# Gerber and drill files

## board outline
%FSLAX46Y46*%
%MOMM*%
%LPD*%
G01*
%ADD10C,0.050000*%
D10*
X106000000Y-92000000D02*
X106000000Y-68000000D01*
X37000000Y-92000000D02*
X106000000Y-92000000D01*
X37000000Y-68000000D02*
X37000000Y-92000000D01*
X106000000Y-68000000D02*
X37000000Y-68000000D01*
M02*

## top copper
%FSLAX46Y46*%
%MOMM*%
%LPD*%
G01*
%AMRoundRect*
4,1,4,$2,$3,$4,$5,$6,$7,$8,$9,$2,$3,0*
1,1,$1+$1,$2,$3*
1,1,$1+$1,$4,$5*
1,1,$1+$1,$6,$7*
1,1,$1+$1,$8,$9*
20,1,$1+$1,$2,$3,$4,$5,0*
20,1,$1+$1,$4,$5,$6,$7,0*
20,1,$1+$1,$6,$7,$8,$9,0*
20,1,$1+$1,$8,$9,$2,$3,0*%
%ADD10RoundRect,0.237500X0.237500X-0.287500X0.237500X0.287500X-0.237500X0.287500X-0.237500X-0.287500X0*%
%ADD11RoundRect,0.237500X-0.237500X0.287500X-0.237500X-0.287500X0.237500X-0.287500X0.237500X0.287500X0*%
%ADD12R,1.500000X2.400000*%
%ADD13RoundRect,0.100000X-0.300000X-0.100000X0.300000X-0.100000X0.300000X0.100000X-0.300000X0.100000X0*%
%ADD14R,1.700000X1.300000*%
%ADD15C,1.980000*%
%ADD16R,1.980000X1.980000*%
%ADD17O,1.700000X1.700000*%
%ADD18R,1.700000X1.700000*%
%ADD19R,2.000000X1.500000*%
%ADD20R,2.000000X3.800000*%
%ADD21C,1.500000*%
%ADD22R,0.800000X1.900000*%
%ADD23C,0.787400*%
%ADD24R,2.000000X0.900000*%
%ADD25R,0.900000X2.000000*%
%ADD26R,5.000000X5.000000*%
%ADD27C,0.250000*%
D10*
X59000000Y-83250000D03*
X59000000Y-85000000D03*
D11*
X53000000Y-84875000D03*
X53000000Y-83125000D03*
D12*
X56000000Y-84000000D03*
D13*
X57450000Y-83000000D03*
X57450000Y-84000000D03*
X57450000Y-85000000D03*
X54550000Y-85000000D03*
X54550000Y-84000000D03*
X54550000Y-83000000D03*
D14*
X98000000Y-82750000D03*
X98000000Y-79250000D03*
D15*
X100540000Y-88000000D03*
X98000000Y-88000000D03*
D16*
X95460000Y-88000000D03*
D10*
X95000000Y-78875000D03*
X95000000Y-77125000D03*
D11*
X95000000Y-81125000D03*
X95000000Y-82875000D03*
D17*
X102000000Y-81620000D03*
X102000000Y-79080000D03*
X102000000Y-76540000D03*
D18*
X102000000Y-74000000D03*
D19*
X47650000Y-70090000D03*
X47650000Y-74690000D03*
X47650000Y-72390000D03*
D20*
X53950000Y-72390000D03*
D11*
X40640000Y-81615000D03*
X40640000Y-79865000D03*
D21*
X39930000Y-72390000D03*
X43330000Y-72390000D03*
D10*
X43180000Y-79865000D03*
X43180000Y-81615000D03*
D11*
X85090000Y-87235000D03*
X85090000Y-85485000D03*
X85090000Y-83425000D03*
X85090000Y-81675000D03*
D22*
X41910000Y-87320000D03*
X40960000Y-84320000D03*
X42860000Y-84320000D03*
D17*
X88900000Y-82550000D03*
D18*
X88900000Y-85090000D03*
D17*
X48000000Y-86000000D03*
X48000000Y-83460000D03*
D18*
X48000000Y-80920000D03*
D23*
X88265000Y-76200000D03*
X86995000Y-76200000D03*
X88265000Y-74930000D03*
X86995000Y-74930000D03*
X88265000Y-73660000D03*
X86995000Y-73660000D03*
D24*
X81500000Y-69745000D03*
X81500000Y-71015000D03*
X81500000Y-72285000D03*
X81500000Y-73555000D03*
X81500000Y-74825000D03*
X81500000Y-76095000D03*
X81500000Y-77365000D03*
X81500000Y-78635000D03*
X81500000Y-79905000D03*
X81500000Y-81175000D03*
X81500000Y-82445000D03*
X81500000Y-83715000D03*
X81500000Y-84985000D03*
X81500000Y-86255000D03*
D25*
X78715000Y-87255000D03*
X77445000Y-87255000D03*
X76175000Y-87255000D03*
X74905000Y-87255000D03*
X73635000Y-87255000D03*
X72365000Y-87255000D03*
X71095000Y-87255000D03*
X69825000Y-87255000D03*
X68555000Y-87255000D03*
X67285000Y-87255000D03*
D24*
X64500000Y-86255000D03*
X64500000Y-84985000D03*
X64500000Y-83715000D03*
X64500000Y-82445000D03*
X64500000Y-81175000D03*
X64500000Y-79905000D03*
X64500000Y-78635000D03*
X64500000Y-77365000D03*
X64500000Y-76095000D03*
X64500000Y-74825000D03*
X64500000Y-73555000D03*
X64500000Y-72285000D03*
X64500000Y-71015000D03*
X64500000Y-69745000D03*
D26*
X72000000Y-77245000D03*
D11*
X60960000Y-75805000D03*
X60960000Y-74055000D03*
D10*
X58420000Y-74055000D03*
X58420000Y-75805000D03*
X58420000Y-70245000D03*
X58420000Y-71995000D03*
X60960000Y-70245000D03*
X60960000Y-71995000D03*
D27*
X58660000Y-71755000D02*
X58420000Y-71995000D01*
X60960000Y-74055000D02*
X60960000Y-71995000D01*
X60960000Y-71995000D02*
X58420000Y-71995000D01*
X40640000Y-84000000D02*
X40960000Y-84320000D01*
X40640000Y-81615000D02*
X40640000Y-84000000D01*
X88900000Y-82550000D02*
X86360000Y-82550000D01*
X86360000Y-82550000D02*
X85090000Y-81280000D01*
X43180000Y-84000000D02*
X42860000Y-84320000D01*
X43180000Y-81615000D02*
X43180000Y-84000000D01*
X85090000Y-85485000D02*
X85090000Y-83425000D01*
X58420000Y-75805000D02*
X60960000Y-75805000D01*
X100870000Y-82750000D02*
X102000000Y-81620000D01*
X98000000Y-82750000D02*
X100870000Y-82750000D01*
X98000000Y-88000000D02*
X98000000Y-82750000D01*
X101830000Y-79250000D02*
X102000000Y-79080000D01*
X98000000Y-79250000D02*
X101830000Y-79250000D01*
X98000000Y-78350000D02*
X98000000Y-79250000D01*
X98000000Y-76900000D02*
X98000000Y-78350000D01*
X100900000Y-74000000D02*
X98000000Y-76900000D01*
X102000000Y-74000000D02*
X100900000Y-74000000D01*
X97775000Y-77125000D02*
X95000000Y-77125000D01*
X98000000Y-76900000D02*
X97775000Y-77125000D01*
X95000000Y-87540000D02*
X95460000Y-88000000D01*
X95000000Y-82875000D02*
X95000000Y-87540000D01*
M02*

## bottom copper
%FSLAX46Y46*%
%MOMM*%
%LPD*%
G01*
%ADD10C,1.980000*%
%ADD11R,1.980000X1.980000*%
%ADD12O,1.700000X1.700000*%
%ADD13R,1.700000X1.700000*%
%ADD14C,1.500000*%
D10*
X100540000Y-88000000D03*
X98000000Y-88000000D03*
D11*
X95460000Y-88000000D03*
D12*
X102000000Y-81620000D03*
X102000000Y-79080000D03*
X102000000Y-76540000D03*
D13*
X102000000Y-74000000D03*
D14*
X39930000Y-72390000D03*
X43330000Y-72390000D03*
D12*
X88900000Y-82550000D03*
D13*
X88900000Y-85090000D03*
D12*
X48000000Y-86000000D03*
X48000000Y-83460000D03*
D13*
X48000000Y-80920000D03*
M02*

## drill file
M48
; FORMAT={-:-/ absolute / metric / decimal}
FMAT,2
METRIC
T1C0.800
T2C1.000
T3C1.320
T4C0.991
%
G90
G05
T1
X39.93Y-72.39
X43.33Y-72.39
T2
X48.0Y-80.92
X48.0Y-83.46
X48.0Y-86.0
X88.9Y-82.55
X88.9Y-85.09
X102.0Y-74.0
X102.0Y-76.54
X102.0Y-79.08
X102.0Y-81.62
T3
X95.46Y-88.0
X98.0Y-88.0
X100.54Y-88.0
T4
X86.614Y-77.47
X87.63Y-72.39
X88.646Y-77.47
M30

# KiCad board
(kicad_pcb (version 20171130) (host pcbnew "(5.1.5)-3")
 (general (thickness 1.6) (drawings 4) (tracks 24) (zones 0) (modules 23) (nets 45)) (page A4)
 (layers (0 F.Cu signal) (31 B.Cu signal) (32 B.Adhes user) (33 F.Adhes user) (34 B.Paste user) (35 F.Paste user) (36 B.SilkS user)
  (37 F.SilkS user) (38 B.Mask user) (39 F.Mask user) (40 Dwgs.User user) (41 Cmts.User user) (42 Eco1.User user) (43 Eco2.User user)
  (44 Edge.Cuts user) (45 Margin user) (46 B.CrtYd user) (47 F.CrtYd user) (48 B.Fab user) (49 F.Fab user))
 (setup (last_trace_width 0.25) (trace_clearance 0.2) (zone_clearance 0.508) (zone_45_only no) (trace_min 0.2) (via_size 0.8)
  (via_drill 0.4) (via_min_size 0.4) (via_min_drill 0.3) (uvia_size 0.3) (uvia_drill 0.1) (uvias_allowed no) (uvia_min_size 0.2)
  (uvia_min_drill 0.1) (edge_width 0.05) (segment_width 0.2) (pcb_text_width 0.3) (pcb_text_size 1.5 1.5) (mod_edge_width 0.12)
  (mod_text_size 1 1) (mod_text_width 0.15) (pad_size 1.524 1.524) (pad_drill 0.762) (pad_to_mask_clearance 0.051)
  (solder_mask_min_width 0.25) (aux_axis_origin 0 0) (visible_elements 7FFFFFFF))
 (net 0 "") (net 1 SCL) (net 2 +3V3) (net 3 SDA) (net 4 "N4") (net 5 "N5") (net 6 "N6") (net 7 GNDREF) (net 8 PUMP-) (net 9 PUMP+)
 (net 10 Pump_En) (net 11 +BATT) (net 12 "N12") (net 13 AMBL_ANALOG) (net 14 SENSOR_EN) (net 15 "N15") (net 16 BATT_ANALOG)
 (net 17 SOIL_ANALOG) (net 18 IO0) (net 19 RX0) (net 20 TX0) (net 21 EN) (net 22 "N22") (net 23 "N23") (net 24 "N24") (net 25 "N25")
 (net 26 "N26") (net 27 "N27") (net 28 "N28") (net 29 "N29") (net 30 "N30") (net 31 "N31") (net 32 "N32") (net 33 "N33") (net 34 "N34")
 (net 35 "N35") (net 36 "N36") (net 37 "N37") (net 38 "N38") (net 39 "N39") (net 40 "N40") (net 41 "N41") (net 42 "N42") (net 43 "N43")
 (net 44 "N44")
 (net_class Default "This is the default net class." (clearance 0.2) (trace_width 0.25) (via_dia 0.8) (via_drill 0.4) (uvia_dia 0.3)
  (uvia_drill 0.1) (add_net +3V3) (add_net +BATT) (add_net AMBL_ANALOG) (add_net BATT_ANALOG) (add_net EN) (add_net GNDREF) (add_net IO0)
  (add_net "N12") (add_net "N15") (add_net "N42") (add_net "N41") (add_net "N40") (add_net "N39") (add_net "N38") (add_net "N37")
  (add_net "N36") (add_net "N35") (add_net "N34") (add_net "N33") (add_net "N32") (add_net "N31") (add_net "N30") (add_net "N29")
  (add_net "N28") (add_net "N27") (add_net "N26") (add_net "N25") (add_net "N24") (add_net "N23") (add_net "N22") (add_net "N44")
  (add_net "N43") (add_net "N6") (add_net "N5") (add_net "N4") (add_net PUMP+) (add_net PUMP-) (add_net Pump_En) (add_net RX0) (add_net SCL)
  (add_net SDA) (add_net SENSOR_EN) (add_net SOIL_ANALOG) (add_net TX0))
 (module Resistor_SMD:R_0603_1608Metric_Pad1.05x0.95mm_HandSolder (layer F.Cu) (at 59 84.125 90)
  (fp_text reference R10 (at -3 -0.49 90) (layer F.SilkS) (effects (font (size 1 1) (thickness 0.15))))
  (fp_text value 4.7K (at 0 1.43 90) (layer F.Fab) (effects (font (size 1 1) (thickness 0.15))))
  (pad 2 smd roundrect (at 0.875 0 90) (size 1.05 0.95) (layers F.Cu F.Paste F.Mask) (roundrect_rratio 0.25) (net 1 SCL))
  (pad 1 smd roundrect (at -0.875 0 90) (size 1.05 0.95) (layers F.Cu F.Paste F.Mask) (roundrect_rratio 0.25) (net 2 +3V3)))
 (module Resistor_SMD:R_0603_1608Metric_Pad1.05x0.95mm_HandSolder (layer F.Cu) (at 53 84 270)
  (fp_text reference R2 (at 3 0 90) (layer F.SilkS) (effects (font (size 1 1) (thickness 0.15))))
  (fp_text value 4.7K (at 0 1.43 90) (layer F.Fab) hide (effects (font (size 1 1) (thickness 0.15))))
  (pad 2 smd roundrect (at 0.875 0 270) (size 1.05 0.95) (layers F.Cu F.Paste F.Mask) (roundrect_rratio 0.25) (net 2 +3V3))
  (pad 1 smd roundrect (at -0.875 0 270) (size 1.05 0.95) (layers F.Cu F.Paste F.Mask) (roundrect_rratio 0.25) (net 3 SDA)))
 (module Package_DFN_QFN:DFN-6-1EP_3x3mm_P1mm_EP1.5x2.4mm (layer F.Cu) (at 56 84)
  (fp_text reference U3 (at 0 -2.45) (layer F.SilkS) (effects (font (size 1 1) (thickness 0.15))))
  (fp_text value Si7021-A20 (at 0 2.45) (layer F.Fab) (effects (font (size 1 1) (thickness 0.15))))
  (pad "" smd roundrect (at 0.375 0.6) (size 0.6 0.97) (layers F.Paste) (roundrect_rratio 0.25))
  (pad "" smd roundrect (at 0.375 -0.6) (size 0.6 0.97) (layers F.Paste) (roundrect_rratio 0.25))
  (pad "" smd roundrect (at -0.375 0.6) (size 0.6 0.97) (layers F.Paste) (roundrect_rratio 0.25))
  (pad "" smd roundrect (at -0.375 -0.6) (size 0.6 0.97) (layers F.Paste) (roundrect_rratio 0.25))
  (pad 7 smd rect (at 0 0) (size 1.5 2.4) (layers F.Cu F.Mask) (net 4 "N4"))
  (pad 6 smd roundrect (at 1.45 -1) (size 0.8 0.4) (layers F.Cu F.Paste F.Mask) (roundrect_rratio 0.25) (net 1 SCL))
  (pad 5 smd roundrect (at 1.45 0) (size 0.8 0.4) (layers F.Cu F.Paste F.Mask) (roundrect_rratio 0.25) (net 2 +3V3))
  (pad 4 smd roundrect (at 1.45 1) (size 0.8 0.4) (layers F.Cu F.Paste F.Mask) (roundrect_rratio 0.25) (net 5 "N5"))
  (pad 3 smd roundrect (at -1.45 1) (size 0.8 0.4) (layers F.Cu F.Paste F.Mask) (roundrect_rratio 0.25) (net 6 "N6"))
  (pad 2 smd roundrect (at -1.45 0) (size 0.8 0.4) (layers F.Cu F.Paste F.Mask) (roundrect_rratio 0.25) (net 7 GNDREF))
  (pad 1 smd roundrect (at -1.45 -1) (size 0.8 0.4) (layers F.Cu F.Paste F.Mask) (roundrect_rratio 0.25) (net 3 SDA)))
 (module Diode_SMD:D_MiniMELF (layer F.Cu) (at 98 81 270)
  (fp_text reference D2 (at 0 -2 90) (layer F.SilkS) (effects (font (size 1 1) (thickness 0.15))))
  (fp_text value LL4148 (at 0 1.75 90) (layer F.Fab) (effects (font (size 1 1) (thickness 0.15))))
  (pad 2 smd rect (at 1.75 0 270) (size 1.3 1.7) (layers F.Cu F.Paste F.Mask) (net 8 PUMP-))
  (pad 1 smd rect (at -1.75 0 270) (size 1.3 1.7) (layers F.Cu F.Paste F.Mask) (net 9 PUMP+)))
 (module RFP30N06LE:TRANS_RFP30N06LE (layer F.Cu) (at 98 88)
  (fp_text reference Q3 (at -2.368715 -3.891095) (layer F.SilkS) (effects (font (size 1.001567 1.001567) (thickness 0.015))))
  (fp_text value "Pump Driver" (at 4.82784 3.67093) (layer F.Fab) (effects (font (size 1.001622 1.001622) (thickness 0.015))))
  (pad 3 thru_hole circle (at 2.54 0) (size 1.98 1.98) (drill 1.32) (layers *.Cu *.Mask) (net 7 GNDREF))
  (pad 2 thru_hole circle (at 0 0) (size 1.98 1.98) (drill 1.32) (layers *.Cu *.Mask) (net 8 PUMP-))
  (pad 1 thru_hole rect (at -2.54 0) (size 1.98 1.98) (drill 1.32) (layers *.Cu *.Mask) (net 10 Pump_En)))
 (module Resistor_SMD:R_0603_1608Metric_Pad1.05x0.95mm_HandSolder (layer F.Cu) (at 95 78 90)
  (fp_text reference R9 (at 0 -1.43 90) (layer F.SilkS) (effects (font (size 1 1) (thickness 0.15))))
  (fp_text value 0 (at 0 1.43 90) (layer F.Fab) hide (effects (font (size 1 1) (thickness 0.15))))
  (pad 1 smd roundrect (at -0.875 0 90) (size 1.05 0.95) (layers F.Cu F.Paste F.Mask) (roundrect_rratio 0.25) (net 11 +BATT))
  (pad 2 smd roundrect (at 0.875 0 90) (size 1.05 0.95) (layers F.Cu F.Paste F.Mask) (roundrect_rratio 0.25) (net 9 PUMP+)))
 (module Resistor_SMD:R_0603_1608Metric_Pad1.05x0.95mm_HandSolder (layer F.Cu) (at 95 82 270)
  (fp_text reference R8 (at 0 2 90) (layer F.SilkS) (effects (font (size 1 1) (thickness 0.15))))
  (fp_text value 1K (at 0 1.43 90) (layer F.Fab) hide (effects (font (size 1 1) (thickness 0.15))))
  (pad 1 smd roundrect (at -0.875 0 270) (size 1.05 0.95) (layers F.Cu F.Paste F.Mask) (roundrect_rratio 0.25) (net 7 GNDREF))
  (pad 2 smd roundrect (at 0.875 0 270) (size 1.05 0.95) (layers F.Cu F.Paste F.Mask) (roundrect_rratio 0.25) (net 10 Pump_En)))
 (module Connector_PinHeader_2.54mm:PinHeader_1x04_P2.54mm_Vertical (layer F.Cu) (at 102 74)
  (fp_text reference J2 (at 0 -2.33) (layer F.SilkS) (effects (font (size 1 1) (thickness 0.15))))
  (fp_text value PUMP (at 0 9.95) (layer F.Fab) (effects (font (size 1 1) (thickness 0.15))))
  (pad 4 thru_hole oval (at 0 7.62) (size 1.7 1.7) (drill 1) (layers *.Cu *.Mask) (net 8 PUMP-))
  (pad 3 thru_hole oval (at 0 5.08) (size 1.7 1.7) (drill 1) (layers *.Cu *.Mask) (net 9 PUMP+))
  (pad 2 thru_hole oval (at 0 2.54) (size 1.7 1.7) (drill 1) (layers *.Cu *.Mask) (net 7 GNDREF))
  (pad 1 thru_hole rect (at 0 0) (size 1.7 1.7) (drill 1) (layers *.Cu *.Mask) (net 9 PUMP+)))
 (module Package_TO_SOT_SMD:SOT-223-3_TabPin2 (layer F.Cu) (at 50.8 72.39)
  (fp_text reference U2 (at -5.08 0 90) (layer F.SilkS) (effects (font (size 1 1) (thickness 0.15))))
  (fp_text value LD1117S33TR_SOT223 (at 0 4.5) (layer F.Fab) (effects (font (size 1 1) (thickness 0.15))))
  (pad 1 smd rect (at -3.15 -2.3) (size 2 1.5) (layers F.Cu F.Paste F.Mask) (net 7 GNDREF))
  (pad 3 smd rect (at -3.15 2.3) (size 2 1.5) (layers F.Cu F.Paste F.Mask) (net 11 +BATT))
  (pad 2 smd rect (at -3.15 0) (size 2 1.5) (layers F.Cu F.Paste F.Mask) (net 2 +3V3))
  (pad 2 smd rect (at 3.15 0) (size 2 3.8) (layers F.Cu F.Paste F.Mask) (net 2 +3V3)))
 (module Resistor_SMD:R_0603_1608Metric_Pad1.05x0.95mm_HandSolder (layer F.Cu) (at 40.64 80.74 270)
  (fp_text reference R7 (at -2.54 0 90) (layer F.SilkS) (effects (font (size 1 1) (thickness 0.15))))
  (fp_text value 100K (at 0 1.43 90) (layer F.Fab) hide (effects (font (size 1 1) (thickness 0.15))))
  (pad 2 smd roundrect (at 0.875 0 270) (size 1.05 0.95) (layers F.Cu F.Paste F.Mask) (roundrect_rratio 0.25) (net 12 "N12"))
  (pad 1 smd roundrect (at -0.875 0 270) (size 1.05 0.95) (layers F.Cu F.Paste F.Mask) (roundrect_rratio 0.25) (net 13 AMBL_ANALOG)))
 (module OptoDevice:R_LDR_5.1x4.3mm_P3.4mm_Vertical (layer F.Cu) (at 43.33 72.39 180)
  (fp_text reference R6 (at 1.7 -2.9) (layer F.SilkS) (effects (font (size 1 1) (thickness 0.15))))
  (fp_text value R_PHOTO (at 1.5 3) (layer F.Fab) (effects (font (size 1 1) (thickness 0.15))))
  (pad 2 thru_hole circle (at 3.4 0 180) (size 1.5 1.5) (drill 0.8) (layers *.Cu *.Mask) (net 13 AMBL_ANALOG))
  (pad 1 thru_hole circle (at 0 0 180) (size 1.5 1.5) (drill 0.8) (layers *.Cu *.Mask) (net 2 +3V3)))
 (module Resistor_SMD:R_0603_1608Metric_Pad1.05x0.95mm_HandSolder (layer F.Cu) (at 43.18 80.74 90)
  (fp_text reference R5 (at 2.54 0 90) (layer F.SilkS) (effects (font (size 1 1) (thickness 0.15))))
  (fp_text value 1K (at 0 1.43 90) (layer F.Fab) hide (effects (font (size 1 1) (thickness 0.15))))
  (pad 2 smd roundrect (at 0.875 0 90) (size 1.05 0.95) (layers F.Cu F.Paste F.Mask) (roundrect_rratio 0.25) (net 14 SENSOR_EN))
  (pad 1 smd roundrect (at -0.875 0 90) (size 1.05 0.95) (layers F.Cu F.Paste F.Mask) (roundrect_rratio 0.25) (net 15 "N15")))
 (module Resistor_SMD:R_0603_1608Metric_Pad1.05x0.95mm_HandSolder (layer F.Cu) (at 85.09 86.36 270)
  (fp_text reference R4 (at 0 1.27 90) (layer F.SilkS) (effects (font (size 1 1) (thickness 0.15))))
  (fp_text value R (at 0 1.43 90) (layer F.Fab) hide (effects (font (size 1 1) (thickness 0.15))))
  (pad 2 smd roundrect (at 0.875 0 270) (size 1.05 0.95) (layers F.Cu F.Paste F.Mask) (roundrect_rratio 0.25) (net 7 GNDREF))
  (pad 1 smd roundrect (at -0.875 0 270) (size 1.05 0.95) (layers F.Cu F.Paste F.Mask) (roundrect_rratio 0.25) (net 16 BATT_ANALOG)))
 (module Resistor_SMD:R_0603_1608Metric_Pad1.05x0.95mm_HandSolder (layer F.Cu) (at 85.09 82.55 270)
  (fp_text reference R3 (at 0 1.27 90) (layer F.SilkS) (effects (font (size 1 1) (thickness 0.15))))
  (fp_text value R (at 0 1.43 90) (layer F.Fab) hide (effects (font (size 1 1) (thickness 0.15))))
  (pad 2 smd roundrect (at 0.875 0 270) (size 1.05 0.95) (layers F.Cu F.Paste F.Mask) (roundrect_rratio 0.25) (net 16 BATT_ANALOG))
  (pad 1 smd roundrect (at -0.875 0 270) (size 1.05 0.95) (layers F.Cu F.Paste F.Mask) (roundrect_rratio 0.25) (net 11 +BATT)))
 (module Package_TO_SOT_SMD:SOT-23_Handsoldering (layer F.Cu) (at 41.91 85.82 270)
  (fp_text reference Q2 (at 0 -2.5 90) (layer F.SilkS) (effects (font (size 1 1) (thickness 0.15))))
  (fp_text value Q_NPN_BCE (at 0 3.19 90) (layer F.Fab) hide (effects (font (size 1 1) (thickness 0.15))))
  (pad 3 smd rect (at 1.5 0 270) (size 1.9 0.8) (layers F.Cu F.Paste F.Mask) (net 7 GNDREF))
  (pad 2 smd rect (at -1.5 0.95 270) (size 1.9 0.8) (layers F.Cu F.Paste F.Mask) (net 12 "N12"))
  (pad 1 smd rect (at -1.5 -0.95 270) (size 1.9 0.8) (layers F.Cu F.Paste F.Mask) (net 15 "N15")))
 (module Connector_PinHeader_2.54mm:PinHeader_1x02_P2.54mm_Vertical (layer F.Cu) (at 88.9 85.09 180)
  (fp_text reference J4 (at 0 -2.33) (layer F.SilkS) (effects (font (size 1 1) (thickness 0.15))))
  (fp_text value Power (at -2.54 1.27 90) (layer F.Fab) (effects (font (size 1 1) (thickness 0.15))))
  (pad 2 thru_hole oval (at 0 2.54 180) (size 1.7 1.7) (drill 1) (layers *.Cu *.Mask) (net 11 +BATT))
  (pad 1 thru_hole rect (at 0 0 180) (size 1.7 1.7) (drill 1) (layers *.Cu *.Mask) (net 7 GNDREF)))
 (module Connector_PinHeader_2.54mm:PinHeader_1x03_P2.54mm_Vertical (layer F.Cu) (at 48 80.92)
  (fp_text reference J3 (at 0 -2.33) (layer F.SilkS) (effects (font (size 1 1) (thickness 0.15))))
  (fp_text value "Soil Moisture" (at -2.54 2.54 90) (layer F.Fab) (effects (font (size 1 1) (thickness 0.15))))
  (pad 3 thru_hole oval (at 0 5.08) (size 1.7 1.7) (drill 1) (layers *.Cu *.Mask) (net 12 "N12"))
  (pad 2 thru_hole oval (at 0 2.54) (size 1.7 1.7) (drill 1) (layers *.Cu *.Mask) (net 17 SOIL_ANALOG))
  (pad 1 thru_hole rect (at 0 0) (size 1.7 1.7) (drill 1) (layers *.Cu *.Mask) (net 2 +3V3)))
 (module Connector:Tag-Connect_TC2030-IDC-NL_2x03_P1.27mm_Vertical (layer F.Cu) (at 87.63 74.93 270)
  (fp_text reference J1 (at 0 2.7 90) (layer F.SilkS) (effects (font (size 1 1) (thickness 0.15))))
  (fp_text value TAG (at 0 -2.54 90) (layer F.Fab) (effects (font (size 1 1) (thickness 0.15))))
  (pad 6 connect circle (at 1.27 -0.635 270) (size 0.7874 0.7874) (layers F.Cu F.Mask) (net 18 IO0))
  (pad 5 connect circle (at 1.27 0.635 270) (size 0.7874 0.7874) (layers F.Cu F.Mask) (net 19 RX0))
  (pad 4 connect circle (at 0 -0.635 270) (size 0.7874 0.7874) (layers F.Cu F.Mask) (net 7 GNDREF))
  (pad 3 connect circle (at 0 0.635 270) (size 0.7874 0.7874) (layers F.Cu F.Mask) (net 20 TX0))
  (pad 2 connect circle (at -1.27 -0.635 270) (size 0.7874 0.7874) (layers F.Cu F.Mask) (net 2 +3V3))
  (pad 1 connect circle (at -1.27 0.635 270) (size 0.7874 0.7874) (layers F.Cu F.Mask) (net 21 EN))
  (pad "" np_thru_hole circle (at -2.54 0 270) (size 0.9906 0.9906) (drill 0.9906) (layers *.Cu *.Mask))
  (pad "" np_thru_hole circle (at 2.54 1.016 270) (size 0.9906 0.9906) (drill 0.9906) (layers *.Cu *.Mask))
  (pad "" np_thru_hole circle (at 2.54 -1.016 270) (size 0.9906 0.9906) (drill 0.9906) (layers *.Cu *.Mask)))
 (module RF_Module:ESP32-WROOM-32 (layer F.Cu) (at 73 78)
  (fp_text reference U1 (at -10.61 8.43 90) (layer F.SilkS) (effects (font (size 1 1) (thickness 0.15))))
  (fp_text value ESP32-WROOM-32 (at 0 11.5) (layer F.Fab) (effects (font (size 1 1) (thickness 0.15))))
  (pad 38 smd rect (at 8.5 -8.255) (size 2 0.9) (layers F.Cu F.Paste F.Mask) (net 7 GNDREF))
  (pad 37 smd rect (at 8.5 -6.985) (size 2 0.9) (layers F.Cu F.Paste F.Mask) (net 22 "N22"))
  (pad 36 smd rect (at 8.5 -5.715) (size 2 0.9) (layers F.Cu F.Paste F.Mask) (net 1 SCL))
  (pad 35 smd rect (at 8.5 -4.445) (size 2 0.9) (layers F.Cu F.Paste F.Mask) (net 20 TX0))
  (pad 34 smd rect (at 8.5 -3.175) (size 2 0.9) (layers F.Cu F.Paste F.Mask) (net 19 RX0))
  (pad 33 smd rect (at 8.5 -1.905) (size 2 0.9) (layers F.Cu F.Paste F.Mask) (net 3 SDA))
  (pad 32 smd rect (at 8.5 -0.635) (size 2 0.9) (layers F.Cu F.Paste F.Mask) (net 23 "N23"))
  (pad 31 smd rect (at 8.5 0.635) (size 2 0.9) (layers F.Cu F.Paste F.Mask) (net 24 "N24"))
  (pad 30 smd rect (at 8.5 1.905) (size 2 0.9) (layers F.Cu F.Paste F.Mask) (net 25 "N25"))
  (pad 29 smd rect (at 8.5 3.175) (size 2 0.9) (layers F.Cu F.Paste F.Mask) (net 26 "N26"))
  (pad 28 smd rect (at 8.5 4.445) (size 2 0.9) (layers F.Cu F.Paste F.Mask) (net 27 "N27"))
  (pad 27 smd rect (at 8.5 5.715) (size 2 0.9) (layers F.Cu F.Paste F.Mask) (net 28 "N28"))
  (pad 26 smd rect (at 8.5 6.985) (size 2 0.9) (layers F.Cu F.Paste F.Mask) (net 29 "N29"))
  (pad 25 smd rect (at 8.5 8.255) (size 2 0.9) (layers F.Cu F.Paste F.Mask) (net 18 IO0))
  (pad 24 smd rect (at 5.715 9.255 90) (size 2 0.9) (layers F.Cu F.Paste F.Mask) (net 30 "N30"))
  (pad 23 smd rect (at 4.445 9.255 90) (size 2 0.9) (layers F.Cu F.Paste F.Mask) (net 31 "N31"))
  (pad 22 smd rect (at 3.175 9.255 90) (size 2 0.9) (layers F.Cu F.Paste F.Mask) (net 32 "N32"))
  (pad 21 smd rect (at 1.905 9.255 90) (size 2 0.9) (layers F.Cu F.Paste F.Mask) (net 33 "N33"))
  (pad 20 smd rect (at 0.635 9.255 90) (size 2 0.9) (layers F.Cu F.Paste F.Mask) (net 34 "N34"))
  (pad 19 smd rect (at -0.635 9.255 90) (size 2 0.9) (layers F.Cu F.Paste F.Mask) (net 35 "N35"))
  (pad 18 smd rect (at -1.905 9.255 90) (size 2 0.9) (layers F.Cu F.Paste F.Mask) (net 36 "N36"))
  (pad 17 smd rect (at -3.175 9.255 90) (size 2 0.9) (layers F.Cu F.Paste F.Mask) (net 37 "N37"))
  (pad 16 smd rect (at -4.445 9.255 90) (size 2 0.9) (layers F.Cu F.Paste F.Mask) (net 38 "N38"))
  (pad 15 smd rect (at -5.715 9.255 90) (size 2 0.9) (layers F.Cu F.Paste F.Mask) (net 7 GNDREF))
  (pad 14 smd rect (at -8.5 8.255) (size 2 0.9) (layers F.Cu F.Paste F.Mask) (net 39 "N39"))
  (pad 13 smd rect (at -8.5 6.985) (size 2 0.9) (layers F.Cu F.Paste F.Mask) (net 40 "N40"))
  (pad 12 smd rect (at -8.5 5.715) (size 2 0.9) (layers F.Cu F.Paste F.Mask) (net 10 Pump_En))
  (pad 11 smd rect (at -8.5 4.445) (size 2 0.9) (layers F.Cu F.Paste F.Mask) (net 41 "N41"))
  (pad 10 smd rect (at -8.5 3.175) (size 2 0.9) (layers F.Cu F.Paste F.Mask) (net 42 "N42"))
  (pad 9 smd rect (at -8.5 1.905) (size 2 0.9) (layers F.Cu F.Paste F.Mask) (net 16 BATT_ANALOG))
  (pad 8 smd rect (at -8.5 0.635) (size 2 0.9) (layers F.Cu F.Paste F.Mask) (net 14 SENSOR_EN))
  (pad 7 smd rect (at -8.5 -0.635) (size 2 0.9) (layers F.Cu F.Paste F.Mask) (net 13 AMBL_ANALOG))
  (pad 6 smd rect (at -8.5 -1.905) (size 2 0.9) (layers F.Cu F.Paste F.Mask) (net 17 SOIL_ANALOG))
  (pad 5 smd rect (at -8.5 -3.175) (size 2 0.9) (layers F.Cu F.Paste F.Mask) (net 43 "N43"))
  (pad 4 smd rect (at -8.5 -4.445) (size 2 0.9) (layers F.Cu F.Paste F.Mask) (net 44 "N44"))
  (pad 3 smd rect (at -8.5 -5.715) (size 2 0.9) (layers F.Cu F.Paste F.Mask) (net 21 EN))
  (pad 2 smd rect (at -8.5 -6.985) (size 2 0.9) (layers F.Cu F.Paste F.Mask) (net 2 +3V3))
  (pad 1 smd rect (at -8.5 -8.255) (size 2 0.9) (layers F.Cu F.Paste F.Mask) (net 7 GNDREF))
  (pad 39 smd rect (at -1 -0.755) (size 5 5) (layers F.Cu F.Paste F.Mask) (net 7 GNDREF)))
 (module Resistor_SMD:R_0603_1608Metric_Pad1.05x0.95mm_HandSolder (layer F.Cu) (at 60.96 74.93 270)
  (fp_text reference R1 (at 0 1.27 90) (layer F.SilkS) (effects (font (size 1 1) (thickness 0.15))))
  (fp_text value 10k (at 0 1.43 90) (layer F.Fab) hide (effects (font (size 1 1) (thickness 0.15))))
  (pad 2 smd roundrect (at 0.875 0 270) (size 1.05 0.95) (layers F.Cu F.Paste F.Mask) (roundrect_rratio 0.25) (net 21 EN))
  (pad 1 smd roundrect (at -0.875 0 270) (size 1.05 0.95) (layers F.Cu F.Paste F.Mask) (roundrect_rratio 0.25) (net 2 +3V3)))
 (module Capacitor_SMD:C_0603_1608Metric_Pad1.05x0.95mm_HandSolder (layer F.Cu) (at 58.42 74.93 90)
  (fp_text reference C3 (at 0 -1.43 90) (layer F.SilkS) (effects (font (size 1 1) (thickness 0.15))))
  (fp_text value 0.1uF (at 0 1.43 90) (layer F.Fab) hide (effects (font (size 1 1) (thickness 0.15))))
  (pad 2 smd roundrect (at 0.875 0 90) (size 1.05 0.95) (layers F.Cu F.Paste F.Mask) (roundrect_rratio 0.25) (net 7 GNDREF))
  (pad 1 smd roundrect (at -0.875 0 90) (size 1.05 0.95) (layers F.Cu F.Paste F.Mask) (roundrect_rratio 0.25) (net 21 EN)))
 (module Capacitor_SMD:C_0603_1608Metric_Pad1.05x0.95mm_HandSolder (layer F.Cu) (at 58.42 71.12 90)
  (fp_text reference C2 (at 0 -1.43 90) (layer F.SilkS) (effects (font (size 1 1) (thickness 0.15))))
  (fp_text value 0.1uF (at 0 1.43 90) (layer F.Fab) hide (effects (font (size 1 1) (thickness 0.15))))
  (pad 2 smd roundrect (at 0.875 0 90) (size 1.05 0.95) (layers F.Cu F.Paste F.Mask) (roundrect_rratio 0.25) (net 7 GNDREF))
  (pad 1 smd roundrect (at -0.875 0 90) (size 1.05 0.95) (layers F.Cu F.Paste F.Mask) (roundrect_rratio 0.25) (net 2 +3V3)))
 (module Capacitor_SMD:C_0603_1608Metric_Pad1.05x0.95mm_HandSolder (layer F.Cu) (at 60.96 71.12 90)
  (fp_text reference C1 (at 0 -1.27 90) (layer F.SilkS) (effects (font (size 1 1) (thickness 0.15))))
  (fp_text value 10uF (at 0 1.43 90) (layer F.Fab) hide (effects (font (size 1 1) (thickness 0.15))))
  (pad 2 smd roundrect (at 0.875 0 90) (size 1.05 0.95) (layers F.Cu F.Paste F.Mask) (roundrect_rratio 0.25) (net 7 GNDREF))
  (pad 1 smd roundrect (at -0.875 0 90) (size 1.05 0.95) (layers F.Cu F.Paste F.Mask) (roundrect_rratio 0.25) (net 2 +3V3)))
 (gr_line (start 106 92) (end 106 68) (layer Edge.Cuts) (width 0.05))
 (gr_line (start 37 92) (end 106 92) (layer Edge.Cuts) (width 0.05))
 (gr_line (start 37 68) (end 37 92) (layer Edge.Cuts) (width 0.05))
 (gr_line (start 106 68) (end 37 68) (layer Edge.Cuts) (width 0.05))
 (segment (start 58.66 71.755) (end 58.42 71.995) (width 0.25) (layer F.Cu) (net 2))
 (segment (start 60.96 74.055) (end 60.96 71.995) (width 0.25) (layer F.Cu) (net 2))
 (segment (start 60.96 71.995) (end 58.42 71.995) (width 0.25) (layer F.Cu) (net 2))
 (segment (start 40.64 84) (end 40.96 84.32) (width 0.25) (layer F.Cu) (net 12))
 (segment (start 40.64 81.615) (end 40.64 84) (width 0.25) (layer F.Cu) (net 12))
 (segment (start 88.9 82.55) (end 86.36 82.55) (width 0.25) (layer F.Cu) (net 11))
 (segment (start 86.36 82.55) (end 85.09 81.28) (width 0.25) (layer F.Cu) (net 11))
 (segment (start 43.18 84) (end 42.86 84.32) (width 0.25) (layer F.Cu) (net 15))
 (segment (start 43.18 81.615) (end 43.18 84) (width 0.25) (layer F.Cu) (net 15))
 (segment (start 85.09 85.485) (end 85.09 83.425) (width 0.25) (layer F.Cu) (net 16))
 (segment (start 58.42 75.805) (end 60.96 75.805) (width 0.25) (layer F.Cu) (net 21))
 (segment (start 100.87 82.75) (end 102 81.62) (width 0.25) (layer F.Cu) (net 8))
 (segment (start 98 82.75) (end 100.87 82.75) (width 0.25) (layer F.Cu) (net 8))
 (segment (start 98 88) (end 98 82.75) (width 0.25) (layer F.Cu) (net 8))
 (segment (start 101.83 79.25) (end 102 79.08) (width 0.25) (layer F.Cu) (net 9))
 (segment (start 98 79.25) (end 101.83 79.25) (width 0.25) (layer F.Cu) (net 9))
 (segment (start 98 78.35) (end 98 79.25) (width 0.25) (layer F.Cu) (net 9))
 (segment (start 98 76.9) (end 98 78.35) (width 0.25) (layer F.Cu) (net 9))
 (segment (start 100.9 74) (end 98 76.9) (width 0.25) (layer F.Cu) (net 9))
 (segment (start 102 74) (end 100.9 74) (width 0.25) (layer F.Cu) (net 9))
 (segment (start 97.775 77.125) (end 95 77.125) (width 0.25) (layer F.Cu) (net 9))
 (segment (start 98 76.9) (end 97.775 77.125) (width 0.25) (layer F.Cu) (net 9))
 (segment (start 95 87.54) (end 95.46 88) (width 0.25) (layer F.Cu) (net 10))
 (segment (start 95 82.875) (end 95 87.54) (width 0.25) (layer F.Cu) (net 10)))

